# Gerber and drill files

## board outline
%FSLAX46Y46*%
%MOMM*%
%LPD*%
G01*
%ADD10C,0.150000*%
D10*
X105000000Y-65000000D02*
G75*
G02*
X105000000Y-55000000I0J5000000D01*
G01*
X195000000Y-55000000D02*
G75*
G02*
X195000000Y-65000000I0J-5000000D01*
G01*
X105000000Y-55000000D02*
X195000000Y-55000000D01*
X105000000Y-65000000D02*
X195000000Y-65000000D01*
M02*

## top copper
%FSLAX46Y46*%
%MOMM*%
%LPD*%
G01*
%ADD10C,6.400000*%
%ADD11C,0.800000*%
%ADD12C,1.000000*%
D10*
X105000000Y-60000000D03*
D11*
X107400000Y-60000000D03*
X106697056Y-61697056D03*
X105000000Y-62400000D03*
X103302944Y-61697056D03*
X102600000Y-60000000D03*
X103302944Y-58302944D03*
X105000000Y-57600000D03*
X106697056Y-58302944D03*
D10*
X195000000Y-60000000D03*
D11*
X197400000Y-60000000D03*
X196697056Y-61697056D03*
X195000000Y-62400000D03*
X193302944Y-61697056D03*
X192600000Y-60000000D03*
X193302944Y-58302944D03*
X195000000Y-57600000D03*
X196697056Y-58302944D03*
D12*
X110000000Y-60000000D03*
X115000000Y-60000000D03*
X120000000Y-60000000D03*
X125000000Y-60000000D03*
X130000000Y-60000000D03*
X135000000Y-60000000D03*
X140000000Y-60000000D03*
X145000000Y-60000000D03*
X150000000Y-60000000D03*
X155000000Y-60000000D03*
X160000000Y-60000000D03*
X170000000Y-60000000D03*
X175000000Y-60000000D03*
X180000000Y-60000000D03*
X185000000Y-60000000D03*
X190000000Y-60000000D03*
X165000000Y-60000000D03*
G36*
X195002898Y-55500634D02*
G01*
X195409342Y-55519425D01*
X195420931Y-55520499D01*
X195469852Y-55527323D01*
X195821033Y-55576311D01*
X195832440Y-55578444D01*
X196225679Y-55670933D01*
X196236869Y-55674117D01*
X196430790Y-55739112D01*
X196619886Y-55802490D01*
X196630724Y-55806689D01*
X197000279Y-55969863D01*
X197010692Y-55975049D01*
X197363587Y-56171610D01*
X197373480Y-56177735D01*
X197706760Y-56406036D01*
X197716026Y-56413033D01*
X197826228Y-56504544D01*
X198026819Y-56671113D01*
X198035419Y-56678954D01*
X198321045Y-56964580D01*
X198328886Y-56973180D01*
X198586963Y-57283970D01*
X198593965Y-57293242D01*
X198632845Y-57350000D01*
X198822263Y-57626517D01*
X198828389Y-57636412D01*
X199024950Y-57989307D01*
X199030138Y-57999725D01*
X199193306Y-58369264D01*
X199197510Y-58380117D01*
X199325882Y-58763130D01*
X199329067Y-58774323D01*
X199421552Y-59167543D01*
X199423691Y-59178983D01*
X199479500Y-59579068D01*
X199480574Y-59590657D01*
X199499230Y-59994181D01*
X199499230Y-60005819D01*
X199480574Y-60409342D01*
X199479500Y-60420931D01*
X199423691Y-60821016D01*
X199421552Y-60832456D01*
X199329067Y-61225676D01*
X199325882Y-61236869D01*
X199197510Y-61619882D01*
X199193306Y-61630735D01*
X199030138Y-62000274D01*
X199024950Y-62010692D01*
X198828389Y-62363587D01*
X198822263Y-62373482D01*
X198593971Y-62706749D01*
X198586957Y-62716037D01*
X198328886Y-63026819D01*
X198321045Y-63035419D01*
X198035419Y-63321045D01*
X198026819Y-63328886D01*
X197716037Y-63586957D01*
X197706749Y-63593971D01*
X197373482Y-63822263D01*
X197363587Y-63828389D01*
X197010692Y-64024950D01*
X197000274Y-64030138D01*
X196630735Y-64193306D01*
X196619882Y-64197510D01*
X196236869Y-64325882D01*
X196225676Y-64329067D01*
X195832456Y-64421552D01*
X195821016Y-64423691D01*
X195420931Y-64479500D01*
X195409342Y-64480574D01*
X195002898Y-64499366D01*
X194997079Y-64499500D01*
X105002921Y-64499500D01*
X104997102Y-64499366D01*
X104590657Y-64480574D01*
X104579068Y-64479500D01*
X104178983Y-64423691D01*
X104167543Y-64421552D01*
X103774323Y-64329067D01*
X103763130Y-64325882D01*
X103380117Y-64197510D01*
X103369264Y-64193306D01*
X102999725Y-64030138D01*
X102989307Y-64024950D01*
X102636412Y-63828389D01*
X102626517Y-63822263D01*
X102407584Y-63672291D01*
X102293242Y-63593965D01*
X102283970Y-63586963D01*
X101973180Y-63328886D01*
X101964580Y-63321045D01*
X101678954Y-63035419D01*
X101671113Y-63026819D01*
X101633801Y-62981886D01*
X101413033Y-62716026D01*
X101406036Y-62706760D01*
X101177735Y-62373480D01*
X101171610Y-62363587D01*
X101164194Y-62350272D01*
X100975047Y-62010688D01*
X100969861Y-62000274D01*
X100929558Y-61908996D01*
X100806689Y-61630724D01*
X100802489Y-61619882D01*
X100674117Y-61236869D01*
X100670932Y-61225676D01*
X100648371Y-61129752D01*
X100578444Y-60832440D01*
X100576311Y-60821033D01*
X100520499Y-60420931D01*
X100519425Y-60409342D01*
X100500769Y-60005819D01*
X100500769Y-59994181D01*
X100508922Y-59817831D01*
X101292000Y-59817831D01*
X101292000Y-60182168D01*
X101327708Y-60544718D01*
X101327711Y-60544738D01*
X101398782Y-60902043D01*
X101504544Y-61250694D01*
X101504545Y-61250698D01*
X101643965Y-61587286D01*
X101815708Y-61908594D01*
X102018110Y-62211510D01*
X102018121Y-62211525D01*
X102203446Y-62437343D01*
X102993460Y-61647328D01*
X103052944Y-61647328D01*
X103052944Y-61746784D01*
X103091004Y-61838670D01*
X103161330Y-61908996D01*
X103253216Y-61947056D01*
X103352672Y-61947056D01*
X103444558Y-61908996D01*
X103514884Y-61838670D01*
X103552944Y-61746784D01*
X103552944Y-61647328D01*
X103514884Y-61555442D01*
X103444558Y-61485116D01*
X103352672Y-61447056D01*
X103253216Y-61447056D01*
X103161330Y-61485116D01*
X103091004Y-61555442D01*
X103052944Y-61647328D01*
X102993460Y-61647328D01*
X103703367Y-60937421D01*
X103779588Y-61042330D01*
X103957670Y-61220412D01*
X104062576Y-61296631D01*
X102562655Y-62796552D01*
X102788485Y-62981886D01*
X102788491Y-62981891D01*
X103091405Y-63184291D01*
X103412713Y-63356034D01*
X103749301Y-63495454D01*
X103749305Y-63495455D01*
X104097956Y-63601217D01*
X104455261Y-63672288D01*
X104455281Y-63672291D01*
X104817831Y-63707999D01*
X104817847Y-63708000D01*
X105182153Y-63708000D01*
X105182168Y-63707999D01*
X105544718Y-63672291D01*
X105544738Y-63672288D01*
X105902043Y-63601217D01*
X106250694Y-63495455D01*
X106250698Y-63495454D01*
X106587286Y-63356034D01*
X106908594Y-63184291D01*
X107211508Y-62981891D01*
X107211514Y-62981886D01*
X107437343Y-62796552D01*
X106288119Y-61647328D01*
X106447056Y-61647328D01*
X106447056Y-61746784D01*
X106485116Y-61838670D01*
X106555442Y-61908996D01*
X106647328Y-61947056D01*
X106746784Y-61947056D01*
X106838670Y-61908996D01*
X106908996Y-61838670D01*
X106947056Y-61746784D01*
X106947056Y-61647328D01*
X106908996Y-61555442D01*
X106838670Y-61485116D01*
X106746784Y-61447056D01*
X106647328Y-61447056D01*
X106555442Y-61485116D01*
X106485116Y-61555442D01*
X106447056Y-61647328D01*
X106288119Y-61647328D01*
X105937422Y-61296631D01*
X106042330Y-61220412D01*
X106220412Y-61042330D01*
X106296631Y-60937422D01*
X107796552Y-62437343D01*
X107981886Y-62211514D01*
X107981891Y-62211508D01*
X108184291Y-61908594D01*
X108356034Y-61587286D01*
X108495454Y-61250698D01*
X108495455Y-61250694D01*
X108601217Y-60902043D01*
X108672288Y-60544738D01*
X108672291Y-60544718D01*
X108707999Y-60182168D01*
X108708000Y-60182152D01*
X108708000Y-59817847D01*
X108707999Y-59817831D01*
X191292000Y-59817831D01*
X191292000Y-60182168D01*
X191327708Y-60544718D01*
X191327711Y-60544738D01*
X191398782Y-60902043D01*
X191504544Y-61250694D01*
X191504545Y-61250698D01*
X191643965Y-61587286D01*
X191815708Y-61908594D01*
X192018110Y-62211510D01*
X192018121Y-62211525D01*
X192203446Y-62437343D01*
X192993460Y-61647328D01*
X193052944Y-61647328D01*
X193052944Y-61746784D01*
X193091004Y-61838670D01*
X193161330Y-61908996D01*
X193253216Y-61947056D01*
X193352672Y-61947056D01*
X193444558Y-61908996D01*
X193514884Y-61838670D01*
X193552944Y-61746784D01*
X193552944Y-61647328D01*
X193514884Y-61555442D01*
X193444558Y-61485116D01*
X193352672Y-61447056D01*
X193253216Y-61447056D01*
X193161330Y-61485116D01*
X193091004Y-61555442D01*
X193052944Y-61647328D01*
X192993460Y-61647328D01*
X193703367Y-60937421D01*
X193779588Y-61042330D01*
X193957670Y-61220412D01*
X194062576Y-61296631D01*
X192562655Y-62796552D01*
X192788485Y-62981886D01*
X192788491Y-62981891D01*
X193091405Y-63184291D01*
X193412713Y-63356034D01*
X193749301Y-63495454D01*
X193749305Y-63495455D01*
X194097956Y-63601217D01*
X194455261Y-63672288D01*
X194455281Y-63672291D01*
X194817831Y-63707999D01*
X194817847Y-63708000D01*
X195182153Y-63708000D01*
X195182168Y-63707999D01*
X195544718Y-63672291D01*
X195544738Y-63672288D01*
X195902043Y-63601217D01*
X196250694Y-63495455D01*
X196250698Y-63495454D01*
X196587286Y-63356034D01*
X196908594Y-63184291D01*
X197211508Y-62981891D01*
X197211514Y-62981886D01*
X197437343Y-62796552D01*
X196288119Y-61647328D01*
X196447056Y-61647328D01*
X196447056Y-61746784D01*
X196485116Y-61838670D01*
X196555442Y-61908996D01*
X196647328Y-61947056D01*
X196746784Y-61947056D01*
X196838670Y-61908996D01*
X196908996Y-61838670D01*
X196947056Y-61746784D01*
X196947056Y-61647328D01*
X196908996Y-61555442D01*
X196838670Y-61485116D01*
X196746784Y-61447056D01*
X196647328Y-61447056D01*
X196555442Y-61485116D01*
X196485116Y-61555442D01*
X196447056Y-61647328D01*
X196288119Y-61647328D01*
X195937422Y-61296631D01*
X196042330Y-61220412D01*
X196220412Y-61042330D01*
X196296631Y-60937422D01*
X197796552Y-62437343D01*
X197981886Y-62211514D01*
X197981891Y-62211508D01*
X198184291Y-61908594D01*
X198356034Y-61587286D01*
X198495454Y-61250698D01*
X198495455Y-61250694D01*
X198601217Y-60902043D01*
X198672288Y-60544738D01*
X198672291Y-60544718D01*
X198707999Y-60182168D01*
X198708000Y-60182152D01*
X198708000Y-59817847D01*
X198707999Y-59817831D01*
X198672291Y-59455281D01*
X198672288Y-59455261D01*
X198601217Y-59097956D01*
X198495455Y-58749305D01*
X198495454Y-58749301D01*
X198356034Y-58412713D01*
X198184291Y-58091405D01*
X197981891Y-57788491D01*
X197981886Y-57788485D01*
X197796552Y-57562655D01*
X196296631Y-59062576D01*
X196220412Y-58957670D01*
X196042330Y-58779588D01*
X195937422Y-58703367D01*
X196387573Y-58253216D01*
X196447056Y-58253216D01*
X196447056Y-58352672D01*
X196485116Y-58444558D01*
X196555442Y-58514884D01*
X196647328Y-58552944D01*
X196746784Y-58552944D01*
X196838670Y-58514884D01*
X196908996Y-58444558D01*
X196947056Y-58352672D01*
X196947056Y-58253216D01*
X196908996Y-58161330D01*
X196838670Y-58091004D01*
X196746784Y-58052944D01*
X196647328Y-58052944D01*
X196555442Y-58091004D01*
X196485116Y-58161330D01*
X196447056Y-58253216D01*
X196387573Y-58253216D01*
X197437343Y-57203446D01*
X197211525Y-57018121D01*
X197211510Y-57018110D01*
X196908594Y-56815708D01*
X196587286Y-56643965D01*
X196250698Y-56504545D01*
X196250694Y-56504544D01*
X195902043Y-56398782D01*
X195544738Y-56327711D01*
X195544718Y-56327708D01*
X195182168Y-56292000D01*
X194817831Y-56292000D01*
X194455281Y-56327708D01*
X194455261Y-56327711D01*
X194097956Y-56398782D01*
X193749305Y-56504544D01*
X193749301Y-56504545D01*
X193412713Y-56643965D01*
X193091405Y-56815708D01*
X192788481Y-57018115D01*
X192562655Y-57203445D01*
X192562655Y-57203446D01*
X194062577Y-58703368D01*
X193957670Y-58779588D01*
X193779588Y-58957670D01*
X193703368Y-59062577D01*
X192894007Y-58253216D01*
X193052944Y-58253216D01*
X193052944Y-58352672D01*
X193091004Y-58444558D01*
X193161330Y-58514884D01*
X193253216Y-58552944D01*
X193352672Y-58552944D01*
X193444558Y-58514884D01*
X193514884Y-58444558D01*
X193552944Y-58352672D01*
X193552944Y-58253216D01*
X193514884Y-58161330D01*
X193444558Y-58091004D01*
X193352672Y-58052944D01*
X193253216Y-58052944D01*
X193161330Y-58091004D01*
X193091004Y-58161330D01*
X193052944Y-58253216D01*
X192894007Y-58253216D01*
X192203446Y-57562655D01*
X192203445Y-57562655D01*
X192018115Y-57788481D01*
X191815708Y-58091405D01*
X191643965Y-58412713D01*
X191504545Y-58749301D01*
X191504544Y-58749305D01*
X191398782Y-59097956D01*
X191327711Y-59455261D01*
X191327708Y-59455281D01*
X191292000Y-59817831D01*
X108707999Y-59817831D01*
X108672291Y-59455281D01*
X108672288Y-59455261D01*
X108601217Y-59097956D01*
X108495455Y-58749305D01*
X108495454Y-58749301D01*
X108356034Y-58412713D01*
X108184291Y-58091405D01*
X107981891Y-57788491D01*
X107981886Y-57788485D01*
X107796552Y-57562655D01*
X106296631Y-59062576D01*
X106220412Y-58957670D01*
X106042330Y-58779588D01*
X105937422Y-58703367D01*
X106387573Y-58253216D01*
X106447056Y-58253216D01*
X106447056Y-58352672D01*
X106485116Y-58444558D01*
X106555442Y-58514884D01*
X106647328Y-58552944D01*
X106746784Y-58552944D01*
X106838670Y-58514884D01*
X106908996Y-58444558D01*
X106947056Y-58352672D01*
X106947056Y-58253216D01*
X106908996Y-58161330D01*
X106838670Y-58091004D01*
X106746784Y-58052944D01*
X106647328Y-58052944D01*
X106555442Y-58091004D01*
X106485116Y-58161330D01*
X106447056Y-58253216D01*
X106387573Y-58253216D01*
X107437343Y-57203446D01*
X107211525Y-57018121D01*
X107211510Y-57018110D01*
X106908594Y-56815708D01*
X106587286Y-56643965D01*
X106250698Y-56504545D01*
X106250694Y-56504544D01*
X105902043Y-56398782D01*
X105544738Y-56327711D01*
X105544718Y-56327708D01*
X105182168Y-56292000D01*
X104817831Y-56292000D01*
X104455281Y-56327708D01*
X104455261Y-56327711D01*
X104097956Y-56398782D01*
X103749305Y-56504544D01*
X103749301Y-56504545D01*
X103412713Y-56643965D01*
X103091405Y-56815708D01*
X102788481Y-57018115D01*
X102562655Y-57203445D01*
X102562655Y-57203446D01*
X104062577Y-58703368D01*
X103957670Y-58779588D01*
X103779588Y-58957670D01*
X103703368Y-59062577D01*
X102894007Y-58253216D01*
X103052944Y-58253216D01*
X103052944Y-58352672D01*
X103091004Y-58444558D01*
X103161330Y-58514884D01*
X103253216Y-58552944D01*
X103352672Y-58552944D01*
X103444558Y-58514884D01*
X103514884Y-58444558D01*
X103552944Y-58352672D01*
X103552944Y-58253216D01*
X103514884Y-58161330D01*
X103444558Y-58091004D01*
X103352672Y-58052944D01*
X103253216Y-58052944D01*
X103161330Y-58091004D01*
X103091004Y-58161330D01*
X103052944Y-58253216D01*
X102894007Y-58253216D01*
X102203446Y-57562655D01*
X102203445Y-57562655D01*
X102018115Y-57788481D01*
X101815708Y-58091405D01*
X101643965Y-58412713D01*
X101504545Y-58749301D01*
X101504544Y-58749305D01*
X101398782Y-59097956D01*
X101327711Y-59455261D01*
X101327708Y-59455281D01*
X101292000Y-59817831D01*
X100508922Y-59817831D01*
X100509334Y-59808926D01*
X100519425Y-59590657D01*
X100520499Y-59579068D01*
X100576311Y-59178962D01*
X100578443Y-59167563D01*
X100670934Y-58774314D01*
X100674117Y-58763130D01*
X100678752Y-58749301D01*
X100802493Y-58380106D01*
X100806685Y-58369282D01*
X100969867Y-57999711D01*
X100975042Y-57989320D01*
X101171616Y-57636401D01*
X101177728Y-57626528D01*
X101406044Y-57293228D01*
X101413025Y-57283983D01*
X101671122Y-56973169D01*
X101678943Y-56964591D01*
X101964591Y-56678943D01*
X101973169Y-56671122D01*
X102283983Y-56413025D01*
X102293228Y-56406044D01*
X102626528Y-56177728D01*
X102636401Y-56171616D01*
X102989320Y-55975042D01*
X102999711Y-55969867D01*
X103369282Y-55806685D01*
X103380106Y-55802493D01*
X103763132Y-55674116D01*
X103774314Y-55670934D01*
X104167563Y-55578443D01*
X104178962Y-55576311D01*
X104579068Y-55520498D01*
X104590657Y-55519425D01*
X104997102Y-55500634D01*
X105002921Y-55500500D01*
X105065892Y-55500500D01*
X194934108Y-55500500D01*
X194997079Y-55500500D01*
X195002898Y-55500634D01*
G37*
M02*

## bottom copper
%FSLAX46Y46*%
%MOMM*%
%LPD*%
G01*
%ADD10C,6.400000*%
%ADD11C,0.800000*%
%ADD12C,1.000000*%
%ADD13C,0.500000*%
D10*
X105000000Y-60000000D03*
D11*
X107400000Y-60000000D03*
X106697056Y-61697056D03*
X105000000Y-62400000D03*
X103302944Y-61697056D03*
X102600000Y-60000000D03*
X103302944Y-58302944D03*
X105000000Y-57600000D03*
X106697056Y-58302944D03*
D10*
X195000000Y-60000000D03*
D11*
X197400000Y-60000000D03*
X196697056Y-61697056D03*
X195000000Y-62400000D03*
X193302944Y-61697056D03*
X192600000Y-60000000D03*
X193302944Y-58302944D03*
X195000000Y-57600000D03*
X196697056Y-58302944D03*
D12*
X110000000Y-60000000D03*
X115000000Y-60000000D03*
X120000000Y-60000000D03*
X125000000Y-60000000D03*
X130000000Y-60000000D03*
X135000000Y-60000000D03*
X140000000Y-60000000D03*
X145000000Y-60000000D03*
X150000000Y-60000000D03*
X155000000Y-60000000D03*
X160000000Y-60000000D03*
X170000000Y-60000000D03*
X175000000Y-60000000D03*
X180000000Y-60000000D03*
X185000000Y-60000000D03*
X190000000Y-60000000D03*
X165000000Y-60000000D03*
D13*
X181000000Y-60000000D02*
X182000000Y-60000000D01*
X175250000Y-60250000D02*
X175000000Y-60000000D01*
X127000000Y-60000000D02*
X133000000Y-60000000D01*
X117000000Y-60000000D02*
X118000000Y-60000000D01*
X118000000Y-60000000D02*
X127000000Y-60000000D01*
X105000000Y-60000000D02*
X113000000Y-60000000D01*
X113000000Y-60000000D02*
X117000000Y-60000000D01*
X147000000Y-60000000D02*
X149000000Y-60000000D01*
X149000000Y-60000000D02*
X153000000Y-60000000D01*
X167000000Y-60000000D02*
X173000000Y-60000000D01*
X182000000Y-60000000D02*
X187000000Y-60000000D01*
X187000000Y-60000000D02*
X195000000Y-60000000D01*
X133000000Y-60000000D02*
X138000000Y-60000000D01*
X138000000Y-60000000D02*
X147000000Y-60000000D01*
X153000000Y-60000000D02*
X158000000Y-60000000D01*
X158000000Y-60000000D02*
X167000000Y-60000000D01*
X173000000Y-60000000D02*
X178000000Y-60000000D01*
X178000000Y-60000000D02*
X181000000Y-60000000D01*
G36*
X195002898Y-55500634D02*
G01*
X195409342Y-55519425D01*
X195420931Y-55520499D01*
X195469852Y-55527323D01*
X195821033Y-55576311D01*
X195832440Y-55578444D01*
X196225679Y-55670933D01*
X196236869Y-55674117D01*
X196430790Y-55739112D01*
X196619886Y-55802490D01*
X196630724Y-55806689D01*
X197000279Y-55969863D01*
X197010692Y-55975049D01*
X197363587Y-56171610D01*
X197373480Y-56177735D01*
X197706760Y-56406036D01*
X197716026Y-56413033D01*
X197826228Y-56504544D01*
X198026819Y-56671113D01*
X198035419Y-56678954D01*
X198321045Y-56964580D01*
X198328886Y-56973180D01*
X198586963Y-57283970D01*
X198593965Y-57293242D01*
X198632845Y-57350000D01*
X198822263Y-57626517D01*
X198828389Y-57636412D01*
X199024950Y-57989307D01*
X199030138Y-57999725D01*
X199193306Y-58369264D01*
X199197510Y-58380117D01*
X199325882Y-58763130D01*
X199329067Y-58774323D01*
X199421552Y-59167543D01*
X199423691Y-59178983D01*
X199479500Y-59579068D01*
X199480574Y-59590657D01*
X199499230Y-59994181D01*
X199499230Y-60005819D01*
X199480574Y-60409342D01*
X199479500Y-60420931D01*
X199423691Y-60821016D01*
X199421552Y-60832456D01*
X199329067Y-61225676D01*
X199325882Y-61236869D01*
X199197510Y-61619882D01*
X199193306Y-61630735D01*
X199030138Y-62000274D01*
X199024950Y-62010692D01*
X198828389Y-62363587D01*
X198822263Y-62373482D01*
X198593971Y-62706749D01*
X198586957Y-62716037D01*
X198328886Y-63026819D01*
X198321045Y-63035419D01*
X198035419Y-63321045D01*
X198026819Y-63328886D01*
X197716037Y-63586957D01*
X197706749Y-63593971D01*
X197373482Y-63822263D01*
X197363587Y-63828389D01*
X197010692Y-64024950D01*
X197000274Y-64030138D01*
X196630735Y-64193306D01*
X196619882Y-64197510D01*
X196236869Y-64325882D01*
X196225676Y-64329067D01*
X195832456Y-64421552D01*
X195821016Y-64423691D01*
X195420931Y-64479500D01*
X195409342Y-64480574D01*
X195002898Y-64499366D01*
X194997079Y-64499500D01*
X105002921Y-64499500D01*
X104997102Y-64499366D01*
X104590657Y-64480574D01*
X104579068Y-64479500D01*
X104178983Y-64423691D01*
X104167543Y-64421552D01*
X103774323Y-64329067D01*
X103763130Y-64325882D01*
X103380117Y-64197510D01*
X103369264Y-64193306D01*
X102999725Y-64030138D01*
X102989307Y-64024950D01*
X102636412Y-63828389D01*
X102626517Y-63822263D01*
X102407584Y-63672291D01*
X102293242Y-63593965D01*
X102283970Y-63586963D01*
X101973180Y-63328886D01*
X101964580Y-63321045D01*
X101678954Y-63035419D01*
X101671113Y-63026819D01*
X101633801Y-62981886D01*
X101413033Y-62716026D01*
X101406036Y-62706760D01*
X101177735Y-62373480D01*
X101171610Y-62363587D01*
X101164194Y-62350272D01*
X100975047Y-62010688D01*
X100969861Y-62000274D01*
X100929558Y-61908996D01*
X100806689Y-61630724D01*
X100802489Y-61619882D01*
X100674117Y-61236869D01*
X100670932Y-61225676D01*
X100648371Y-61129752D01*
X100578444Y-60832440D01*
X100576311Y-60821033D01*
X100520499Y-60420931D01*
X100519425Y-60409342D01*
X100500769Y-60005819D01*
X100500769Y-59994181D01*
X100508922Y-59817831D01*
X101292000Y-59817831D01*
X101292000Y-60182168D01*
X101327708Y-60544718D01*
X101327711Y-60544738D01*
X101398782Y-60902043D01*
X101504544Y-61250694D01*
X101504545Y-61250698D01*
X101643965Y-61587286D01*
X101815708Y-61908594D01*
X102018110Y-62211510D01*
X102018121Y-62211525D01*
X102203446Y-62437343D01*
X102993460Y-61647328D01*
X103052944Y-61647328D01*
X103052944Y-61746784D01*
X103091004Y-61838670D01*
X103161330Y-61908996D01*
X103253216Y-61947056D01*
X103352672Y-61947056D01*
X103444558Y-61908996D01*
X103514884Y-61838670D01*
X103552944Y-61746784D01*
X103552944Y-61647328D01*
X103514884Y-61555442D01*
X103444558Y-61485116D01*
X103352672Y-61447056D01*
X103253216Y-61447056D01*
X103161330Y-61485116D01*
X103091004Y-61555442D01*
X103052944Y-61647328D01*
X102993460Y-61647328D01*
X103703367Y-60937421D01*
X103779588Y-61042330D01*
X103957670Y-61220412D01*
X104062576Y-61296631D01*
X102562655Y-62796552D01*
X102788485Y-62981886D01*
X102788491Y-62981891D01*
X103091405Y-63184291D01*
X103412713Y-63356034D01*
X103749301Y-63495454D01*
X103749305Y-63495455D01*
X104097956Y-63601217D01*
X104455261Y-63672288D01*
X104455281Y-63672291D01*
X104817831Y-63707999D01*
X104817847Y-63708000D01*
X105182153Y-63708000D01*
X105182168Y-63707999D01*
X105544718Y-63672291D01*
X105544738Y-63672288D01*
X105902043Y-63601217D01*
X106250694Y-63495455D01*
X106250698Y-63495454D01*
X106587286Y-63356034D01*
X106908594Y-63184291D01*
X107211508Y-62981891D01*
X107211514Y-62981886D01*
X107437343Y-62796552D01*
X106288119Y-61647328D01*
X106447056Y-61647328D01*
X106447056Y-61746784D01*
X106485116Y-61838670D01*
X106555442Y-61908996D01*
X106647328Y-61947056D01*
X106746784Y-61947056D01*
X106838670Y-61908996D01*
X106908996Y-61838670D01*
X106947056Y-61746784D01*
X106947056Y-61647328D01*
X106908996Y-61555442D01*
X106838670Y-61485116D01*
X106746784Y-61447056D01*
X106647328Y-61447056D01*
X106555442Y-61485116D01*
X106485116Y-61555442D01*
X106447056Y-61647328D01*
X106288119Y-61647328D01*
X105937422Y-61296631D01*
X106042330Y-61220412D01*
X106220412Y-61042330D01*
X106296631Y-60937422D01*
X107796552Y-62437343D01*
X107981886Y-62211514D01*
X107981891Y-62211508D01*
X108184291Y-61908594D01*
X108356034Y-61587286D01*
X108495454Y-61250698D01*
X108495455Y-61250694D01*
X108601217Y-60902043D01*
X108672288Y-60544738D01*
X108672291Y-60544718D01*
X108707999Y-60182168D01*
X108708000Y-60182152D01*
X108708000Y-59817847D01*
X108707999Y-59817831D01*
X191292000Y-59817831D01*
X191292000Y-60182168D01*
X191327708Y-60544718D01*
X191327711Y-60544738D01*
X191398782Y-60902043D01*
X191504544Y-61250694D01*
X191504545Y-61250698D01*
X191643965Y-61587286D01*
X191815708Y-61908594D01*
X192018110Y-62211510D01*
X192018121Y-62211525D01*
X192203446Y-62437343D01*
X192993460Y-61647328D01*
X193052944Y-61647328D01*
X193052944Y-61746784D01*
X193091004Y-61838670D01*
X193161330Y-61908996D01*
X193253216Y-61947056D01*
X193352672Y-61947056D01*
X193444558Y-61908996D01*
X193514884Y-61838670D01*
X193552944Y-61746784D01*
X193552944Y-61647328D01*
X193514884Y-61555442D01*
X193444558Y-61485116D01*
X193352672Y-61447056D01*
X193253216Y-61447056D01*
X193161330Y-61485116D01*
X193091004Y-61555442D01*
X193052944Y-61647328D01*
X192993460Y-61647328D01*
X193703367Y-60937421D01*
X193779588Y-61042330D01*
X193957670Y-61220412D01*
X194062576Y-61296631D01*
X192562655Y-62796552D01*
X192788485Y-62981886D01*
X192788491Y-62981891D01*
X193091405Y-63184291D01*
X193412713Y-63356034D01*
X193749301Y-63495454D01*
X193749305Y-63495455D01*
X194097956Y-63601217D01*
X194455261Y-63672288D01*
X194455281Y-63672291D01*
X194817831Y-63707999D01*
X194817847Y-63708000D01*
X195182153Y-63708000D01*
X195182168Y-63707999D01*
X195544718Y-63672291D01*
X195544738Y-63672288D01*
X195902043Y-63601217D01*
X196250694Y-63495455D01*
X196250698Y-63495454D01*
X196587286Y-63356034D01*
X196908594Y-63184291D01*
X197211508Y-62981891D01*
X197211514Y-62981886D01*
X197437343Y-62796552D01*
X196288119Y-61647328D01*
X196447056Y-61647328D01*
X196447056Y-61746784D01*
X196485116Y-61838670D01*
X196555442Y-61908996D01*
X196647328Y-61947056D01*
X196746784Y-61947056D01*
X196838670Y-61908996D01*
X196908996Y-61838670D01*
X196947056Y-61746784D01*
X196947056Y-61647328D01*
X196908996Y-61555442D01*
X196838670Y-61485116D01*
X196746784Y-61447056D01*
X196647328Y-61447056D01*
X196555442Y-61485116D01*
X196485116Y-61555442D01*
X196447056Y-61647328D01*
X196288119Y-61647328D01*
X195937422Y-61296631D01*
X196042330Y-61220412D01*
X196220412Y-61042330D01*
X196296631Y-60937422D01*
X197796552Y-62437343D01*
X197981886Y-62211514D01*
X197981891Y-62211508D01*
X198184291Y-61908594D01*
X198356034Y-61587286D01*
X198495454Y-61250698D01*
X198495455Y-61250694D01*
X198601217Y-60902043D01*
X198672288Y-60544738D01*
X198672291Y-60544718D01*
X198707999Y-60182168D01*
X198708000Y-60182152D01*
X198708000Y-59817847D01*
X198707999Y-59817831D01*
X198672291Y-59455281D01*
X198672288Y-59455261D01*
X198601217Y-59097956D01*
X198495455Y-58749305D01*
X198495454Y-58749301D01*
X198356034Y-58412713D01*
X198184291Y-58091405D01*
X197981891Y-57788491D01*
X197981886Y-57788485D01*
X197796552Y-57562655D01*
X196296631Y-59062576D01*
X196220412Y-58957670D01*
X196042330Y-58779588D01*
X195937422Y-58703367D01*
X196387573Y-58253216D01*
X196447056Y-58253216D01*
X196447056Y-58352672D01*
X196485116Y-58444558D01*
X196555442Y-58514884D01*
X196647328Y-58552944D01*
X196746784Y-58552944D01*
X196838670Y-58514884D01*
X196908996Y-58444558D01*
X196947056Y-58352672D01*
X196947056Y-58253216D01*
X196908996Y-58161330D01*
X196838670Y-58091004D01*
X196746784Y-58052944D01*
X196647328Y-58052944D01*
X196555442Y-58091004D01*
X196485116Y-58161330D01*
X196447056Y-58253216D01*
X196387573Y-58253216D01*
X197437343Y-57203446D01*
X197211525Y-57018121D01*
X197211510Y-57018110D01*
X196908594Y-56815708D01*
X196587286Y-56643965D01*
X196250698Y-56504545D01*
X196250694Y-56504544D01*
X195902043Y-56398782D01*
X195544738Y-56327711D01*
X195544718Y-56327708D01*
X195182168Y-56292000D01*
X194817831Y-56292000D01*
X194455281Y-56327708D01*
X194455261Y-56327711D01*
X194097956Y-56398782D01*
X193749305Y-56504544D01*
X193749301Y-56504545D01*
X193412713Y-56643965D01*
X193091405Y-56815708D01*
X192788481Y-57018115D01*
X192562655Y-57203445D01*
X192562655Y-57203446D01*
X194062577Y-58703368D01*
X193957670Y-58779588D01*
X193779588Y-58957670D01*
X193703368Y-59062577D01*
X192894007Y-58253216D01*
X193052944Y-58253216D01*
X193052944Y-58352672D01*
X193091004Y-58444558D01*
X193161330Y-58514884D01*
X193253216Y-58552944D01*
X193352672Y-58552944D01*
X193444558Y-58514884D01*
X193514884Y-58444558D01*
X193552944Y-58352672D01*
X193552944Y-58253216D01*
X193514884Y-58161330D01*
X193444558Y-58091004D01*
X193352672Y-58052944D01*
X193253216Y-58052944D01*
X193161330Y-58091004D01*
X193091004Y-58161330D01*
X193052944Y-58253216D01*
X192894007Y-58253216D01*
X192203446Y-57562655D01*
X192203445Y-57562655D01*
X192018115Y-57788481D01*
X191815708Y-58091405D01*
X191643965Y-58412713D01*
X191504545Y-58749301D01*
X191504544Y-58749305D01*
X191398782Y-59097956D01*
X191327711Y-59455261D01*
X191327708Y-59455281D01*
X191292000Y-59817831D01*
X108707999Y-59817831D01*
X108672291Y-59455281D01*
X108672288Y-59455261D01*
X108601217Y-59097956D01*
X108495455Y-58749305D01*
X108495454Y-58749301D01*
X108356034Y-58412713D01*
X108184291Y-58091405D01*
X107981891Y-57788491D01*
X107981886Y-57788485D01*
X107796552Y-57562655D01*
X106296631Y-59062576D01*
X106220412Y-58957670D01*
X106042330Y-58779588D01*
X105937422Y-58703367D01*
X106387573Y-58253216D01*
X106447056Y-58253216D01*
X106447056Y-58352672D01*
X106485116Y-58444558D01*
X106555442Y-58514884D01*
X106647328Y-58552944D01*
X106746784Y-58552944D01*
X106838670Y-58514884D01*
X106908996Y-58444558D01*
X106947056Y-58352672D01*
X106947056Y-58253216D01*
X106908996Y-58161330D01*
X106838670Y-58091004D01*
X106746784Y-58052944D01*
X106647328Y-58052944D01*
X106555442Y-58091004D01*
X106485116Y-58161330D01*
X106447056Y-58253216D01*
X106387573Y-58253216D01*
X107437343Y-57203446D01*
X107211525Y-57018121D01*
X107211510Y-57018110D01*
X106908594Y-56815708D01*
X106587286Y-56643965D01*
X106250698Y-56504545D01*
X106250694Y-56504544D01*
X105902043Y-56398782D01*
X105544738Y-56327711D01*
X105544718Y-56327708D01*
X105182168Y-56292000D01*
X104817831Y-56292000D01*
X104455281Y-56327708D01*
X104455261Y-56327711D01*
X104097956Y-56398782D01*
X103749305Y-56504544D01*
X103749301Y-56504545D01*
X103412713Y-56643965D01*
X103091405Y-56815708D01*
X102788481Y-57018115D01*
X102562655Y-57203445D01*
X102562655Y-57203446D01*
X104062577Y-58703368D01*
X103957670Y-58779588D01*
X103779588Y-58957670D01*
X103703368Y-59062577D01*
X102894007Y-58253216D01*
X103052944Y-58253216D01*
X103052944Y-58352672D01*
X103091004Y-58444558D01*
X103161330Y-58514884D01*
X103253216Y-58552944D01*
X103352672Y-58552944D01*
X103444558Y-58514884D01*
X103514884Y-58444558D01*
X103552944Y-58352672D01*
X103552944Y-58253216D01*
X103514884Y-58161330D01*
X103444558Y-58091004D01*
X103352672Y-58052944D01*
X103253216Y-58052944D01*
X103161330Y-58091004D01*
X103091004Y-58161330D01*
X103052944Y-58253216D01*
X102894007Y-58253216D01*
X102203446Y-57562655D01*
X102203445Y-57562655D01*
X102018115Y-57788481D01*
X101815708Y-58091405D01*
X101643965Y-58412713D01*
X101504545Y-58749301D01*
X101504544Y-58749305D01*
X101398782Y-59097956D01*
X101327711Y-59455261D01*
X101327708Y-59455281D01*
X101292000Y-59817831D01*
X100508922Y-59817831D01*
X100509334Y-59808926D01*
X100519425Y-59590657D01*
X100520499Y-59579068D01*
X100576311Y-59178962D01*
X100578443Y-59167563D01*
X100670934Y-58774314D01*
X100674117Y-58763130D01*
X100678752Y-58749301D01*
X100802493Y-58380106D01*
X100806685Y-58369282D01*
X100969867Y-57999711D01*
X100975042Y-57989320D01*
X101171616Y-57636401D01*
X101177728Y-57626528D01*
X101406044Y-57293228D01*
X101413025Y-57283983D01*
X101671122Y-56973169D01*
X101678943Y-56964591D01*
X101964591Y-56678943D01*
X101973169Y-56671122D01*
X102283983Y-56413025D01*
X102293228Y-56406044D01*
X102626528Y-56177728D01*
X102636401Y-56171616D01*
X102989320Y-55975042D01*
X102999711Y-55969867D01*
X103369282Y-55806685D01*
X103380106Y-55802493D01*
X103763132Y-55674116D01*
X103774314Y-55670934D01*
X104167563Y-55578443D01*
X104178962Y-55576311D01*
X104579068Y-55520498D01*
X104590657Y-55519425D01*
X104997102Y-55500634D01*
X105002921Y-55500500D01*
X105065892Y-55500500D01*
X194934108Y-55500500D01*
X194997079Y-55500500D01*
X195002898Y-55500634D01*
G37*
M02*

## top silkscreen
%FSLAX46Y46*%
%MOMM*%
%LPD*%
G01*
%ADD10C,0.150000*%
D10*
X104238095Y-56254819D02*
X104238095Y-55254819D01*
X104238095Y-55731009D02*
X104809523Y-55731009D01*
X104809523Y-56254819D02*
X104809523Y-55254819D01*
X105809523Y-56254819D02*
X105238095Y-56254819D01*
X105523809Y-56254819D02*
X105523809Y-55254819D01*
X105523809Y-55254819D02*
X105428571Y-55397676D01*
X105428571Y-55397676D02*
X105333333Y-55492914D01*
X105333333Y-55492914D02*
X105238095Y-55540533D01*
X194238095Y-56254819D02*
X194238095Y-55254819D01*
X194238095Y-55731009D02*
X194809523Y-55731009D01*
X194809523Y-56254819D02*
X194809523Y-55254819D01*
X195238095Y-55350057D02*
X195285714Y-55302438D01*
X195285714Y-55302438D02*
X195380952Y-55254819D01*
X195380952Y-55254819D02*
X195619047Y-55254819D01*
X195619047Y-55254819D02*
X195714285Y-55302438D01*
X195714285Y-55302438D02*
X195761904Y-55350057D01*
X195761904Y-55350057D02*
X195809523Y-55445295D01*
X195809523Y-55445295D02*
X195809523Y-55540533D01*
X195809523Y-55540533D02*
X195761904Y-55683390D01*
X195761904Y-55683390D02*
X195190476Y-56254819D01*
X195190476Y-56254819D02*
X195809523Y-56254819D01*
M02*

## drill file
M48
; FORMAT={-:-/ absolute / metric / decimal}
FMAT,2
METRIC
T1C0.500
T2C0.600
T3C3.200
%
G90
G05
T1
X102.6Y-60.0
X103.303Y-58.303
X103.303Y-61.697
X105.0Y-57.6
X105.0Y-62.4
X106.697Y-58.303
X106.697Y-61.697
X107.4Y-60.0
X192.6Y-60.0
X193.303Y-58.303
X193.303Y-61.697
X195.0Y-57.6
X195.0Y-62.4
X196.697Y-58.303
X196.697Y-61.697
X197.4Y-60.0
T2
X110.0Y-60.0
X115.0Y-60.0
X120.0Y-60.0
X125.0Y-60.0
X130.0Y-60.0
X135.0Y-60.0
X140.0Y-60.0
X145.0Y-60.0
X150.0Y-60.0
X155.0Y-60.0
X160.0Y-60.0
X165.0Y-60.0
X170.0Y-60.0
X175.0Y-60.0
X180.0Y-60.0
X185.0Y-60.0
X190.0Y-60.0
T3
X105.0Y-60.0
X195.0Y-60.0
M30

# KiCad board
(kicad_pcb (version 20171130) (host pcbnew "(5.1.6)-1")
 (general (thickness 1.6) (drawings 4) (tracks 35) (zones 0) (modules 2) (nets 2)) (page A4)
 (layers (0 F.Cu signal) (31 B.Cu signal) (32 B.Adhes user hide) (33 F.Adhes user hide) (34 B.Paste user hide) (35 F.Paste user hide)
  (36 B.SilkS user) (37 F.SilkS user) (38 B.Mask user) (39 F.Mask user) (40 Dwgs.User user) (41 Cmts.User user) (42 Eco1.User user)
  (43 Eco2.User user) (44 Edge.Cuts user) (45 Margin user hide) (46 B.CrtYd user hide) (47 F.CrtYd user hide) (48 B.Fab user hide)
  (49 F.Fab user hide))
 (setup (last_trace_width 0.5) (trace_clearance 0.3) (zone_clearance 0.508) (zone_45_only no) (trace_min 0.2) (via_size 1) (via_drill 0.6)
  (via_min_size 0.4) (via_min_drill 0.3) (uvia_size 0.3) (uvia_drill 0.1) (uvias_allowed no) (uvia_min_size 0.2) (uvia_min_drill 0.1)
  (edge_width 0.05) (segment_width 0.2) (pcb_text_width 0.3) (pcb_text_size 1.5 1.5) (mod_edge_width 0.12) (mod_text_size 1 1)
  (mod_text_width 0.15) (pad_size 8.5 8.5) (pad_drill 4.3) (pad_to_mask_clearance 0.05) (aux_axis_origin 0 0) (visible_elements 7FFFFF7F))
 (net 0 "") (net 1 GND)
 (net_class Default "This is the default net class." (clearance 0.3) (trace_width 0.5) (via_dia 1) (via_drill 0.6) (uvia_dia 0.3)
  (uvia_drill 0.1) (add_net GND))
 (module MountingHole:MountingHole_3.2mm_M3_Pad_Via (layer F.Cu) (at 105 60)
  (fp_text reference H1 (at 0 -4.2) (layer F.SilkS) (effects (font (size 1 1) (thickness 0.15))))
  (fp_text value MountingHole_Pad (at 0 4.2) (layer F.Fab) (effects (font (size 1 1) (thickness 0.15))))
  (pad 1 thru_hole circle (at 0 0) (size 6.4 6.4) (drill 3.2) (layers *.Cu *.Mask) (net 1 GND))
  (pad 1 thru_hole circle (at 2.4 0) (size 0.8 0.8) (drill 0.5) (layers *.Cu *.Mask) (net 1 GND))
  (pad 1 thru_hole circle (at 1.697056 1.697056) (size 0.8 0.8) (drill 0.5) (layers *.Cu *.Mask) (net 1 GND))
  (pad 1 thru_hole circle (at 0 2.4) (size 0.8 0.8) (drill 0.5) (layers *.Cu *.Mask) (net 1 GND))
  (pad 1 thru_hole circle (at -1.697056 1.697056) (size 0.8 0.8) (drill 0.5) (layers *.Cu *.Mask) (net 1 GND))
  (pad 1 thru_hole circle (at -2.4 0) (size 0.8 0.8) (drill 0.5) (layers *.Cu *.Mask) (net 1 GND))
  (pad 1 thru_hole circle (at -1.697056 -1.697056) (size 0.8 0.8) (drill 0.5) (layers *.Cu *.Mask) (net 1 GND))
  (pad 1 thru_hole circle (at 0 -2.4) (size 0.8 0.8) (drill 0.5) (layers *.Cu *.Mask) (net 1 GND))
  (pad 1 thru_hole circle (at 1.697056 -1.697056) (size 0.8 0.8) (drill 0.5) (layers *.Cu *.Mask) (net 1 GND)))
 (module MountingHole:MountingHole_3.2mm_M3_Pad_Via (layer F.Cu) (at 195 60)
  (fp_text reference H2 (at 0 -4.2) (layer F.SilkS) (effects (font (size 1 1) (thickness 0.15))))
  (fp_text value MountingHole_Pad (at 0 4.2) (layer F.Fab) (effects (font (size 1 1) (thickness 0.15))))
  (pad 1 thru_hole circle (at 0 0) (size 6.4 6.4) (drill 3.2) (layers *.Cu *.Mask) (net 1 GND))
  (pad 1 thru_hole circle (at 2.4 0) (size 0.8 0.8) (drill 0.5) (layers *.Cu *.Mask) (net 1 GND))
  (pad 1 thru_hole circle (at 1.697056 1.697056) (size 0.8 0.8) (drill 0.5) (layers *.Cu *.Mask) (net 1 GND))
  (pad 1 thru_hole circle (at 0 2.4) (size 0.8 0.8) (drill 0.5) (layers *.Cu *.Mask) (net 1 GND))
  (pad 1 thru_hole circle (at -1.697056 1.697056) (size 0.8 0.8) (drill 0.5) (layers *.Cu *.Mask) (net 1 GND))
  (pad 1 thru_hole circle (at -2.4 0) (size 0.8 0.8) (drill 0.5) (layers *.Cu *.Mask) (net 1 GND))
  (pad 1 thru_hole circle (at -1.697056 -1.697056) (size 0.8 0.8) (drill 0.5) (layers *.Cu *.Mask) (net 1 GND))
  (pad 1 thru_hole circle (at 0 -2.4) (size 0.8 0.8) (drill 0.5) (layers *.Cu *.Mask) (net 1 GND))
  (pad 1 thru_hole circle (at 1.697056 -1.697056) (size 0.8 0.8) (drill 0.5) (layers *.Cu *.Mask) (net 1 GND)))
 (gr_arc (start 105 60) (end 105 55) (angle -180) (layer Edge.Cuts) (width 0.15))
 (gr_arc (start 195 60) (end 195 65) (angle -180) (layer Edge.Cuts) (width 0.15))
 (gr_line (start 105 55) (end 195 55) (layer Edge.Cuts) (width 0.15))
 (gr_line (start 105 65) (end 195 65) (layer Edge.Cuts) (width 0.15))
 (via (at 110 60) (size 1) (drill 0.6) (layers F.Cu B.Cu) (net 1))
 (via (at 115 60) (size 1) (drill 0.6) (layers F.Cu B.Cu) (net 1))
 (via (at 120 60) (size 1) (drill 0.6) (layers F.Cu B.Cu) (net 1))
 (via (at 125 60) (size 1) (drill 0.6) (layers F.Cu B.Cu) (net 1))
 (via (at 130 60) (size 1) (drill 0.6) (layers F.Cu B.Cu) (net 1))
 (via (at 135 60) (size 1) (drill 0.6) (layers F.Cu B.Cu) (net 1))
 (via (at 140 60) (size 1) (drill 0.6) (layers F.Cu B.Cu) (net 1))
 (via (at 145 60) (size 1) (drill 0.6) (layers F.Cu B.Cu) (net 1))
 (via (at 150 60) (size 1) (drill 0.6) (layers F.Cu B.Cu) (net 1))
 (via (at 155 60) (size 1) (drill 0.6) (layers F.Cu B.Cu) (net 1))
 (via (at 160 60) (size 1) (drill 0.6) (layers F.Cu B.Cu) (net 1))
 (via (at 170 60) (size 1) (drill 0.6) (layers F.Cu B.Cu) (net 1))
 (via (at 175 60) (size 1) (drill 0.6) (layers F.Cu B.Cu) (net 1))
 (via (at 180 60) (size 1) (drill 0.6) (layers F.Cu B.Cu) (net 1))
 (via (at 185 60) (size 1) (drill 0.6) (layers F.Cu B.Cu) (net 1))
 (via (at 190 60) (size 1) (drill 0.6) (layers F.Cu B.Cu) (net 1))
 (segment (start 181 60) (end 182 60) (width 0.5) (layer B.Cu) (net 1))
 (segment (start 175.25 60.25) (end 175 60) (width 0.5) (layer B.Cu) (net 1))
 (via (at 165 60) (size 1) (drill 0.6) (layers F.Cu B.Cu) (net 1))
 (segment (start 127 60) (end 133 60) (width 0.5) (layer B.Cu) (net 1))
 (segment (start 117 60) (end 118 60) (width 0.5) (layer B.Cu) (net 1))
 (segment (start 118 60) (end 127 60) (width 0.5) (layer B.Cu) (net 1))
 (segment (start 105 60) (end 113 60) (width 0.5) (layer B.Cu) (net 1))
 (segment (start 113 60) (end 117 60) (width 0.5) (layer B.Cu) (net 1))
 (segment (start 147 60) (end 149 60) (width 0.5) (layer B.Cu) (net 1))
 (segment (start 149 60) (end 153 60) (width 0.5) (layer B.Cu) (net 1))
 (segment (start 167 60) (end 173 60) (width 0.5) (layer B.Cu) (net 1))
 (segment (start 182 60) (end 187 60) (width 0.5) (layer B.Cu) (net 1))
 (segment (start 187 60) (end 195 60) (width 0.5) (layer B.Cu) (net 1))
 (segment (start 133 60) (end 138 60) (width 0.5) (layer B.Cu) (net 1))
 (segment (start 138 60) (end 147 60) (width 0.5) (layer B.Cu) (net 1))
 (segment (start 153 60) (end 158 60) (width 0.5) (layer B.Cu) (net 1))
 (segment (start 158 60) (end 167 60) (width 0.5) (layer B.Cu) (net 1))
 (segment (start 173 60) (end 178 60) (width 0.5) (layer B.Cu) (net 1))
 (segment (start 178 60) (end 181 60) (width 0.5) (layer B.Cu) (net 1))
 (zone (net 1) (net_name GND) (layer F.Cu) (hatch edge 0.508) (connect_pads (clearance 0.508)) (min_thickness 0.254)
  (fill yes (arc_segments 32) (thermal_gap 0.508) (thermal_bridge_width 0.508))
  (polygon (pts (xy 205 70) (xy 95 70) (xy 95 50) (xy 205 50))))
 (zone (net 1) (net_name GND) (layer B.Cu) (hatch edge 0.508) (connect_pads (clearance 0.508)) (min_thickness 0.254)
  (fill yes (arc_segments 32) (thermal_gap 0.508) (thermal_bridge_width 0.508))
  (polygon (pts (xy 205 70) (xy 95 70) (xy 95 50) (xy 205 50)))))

